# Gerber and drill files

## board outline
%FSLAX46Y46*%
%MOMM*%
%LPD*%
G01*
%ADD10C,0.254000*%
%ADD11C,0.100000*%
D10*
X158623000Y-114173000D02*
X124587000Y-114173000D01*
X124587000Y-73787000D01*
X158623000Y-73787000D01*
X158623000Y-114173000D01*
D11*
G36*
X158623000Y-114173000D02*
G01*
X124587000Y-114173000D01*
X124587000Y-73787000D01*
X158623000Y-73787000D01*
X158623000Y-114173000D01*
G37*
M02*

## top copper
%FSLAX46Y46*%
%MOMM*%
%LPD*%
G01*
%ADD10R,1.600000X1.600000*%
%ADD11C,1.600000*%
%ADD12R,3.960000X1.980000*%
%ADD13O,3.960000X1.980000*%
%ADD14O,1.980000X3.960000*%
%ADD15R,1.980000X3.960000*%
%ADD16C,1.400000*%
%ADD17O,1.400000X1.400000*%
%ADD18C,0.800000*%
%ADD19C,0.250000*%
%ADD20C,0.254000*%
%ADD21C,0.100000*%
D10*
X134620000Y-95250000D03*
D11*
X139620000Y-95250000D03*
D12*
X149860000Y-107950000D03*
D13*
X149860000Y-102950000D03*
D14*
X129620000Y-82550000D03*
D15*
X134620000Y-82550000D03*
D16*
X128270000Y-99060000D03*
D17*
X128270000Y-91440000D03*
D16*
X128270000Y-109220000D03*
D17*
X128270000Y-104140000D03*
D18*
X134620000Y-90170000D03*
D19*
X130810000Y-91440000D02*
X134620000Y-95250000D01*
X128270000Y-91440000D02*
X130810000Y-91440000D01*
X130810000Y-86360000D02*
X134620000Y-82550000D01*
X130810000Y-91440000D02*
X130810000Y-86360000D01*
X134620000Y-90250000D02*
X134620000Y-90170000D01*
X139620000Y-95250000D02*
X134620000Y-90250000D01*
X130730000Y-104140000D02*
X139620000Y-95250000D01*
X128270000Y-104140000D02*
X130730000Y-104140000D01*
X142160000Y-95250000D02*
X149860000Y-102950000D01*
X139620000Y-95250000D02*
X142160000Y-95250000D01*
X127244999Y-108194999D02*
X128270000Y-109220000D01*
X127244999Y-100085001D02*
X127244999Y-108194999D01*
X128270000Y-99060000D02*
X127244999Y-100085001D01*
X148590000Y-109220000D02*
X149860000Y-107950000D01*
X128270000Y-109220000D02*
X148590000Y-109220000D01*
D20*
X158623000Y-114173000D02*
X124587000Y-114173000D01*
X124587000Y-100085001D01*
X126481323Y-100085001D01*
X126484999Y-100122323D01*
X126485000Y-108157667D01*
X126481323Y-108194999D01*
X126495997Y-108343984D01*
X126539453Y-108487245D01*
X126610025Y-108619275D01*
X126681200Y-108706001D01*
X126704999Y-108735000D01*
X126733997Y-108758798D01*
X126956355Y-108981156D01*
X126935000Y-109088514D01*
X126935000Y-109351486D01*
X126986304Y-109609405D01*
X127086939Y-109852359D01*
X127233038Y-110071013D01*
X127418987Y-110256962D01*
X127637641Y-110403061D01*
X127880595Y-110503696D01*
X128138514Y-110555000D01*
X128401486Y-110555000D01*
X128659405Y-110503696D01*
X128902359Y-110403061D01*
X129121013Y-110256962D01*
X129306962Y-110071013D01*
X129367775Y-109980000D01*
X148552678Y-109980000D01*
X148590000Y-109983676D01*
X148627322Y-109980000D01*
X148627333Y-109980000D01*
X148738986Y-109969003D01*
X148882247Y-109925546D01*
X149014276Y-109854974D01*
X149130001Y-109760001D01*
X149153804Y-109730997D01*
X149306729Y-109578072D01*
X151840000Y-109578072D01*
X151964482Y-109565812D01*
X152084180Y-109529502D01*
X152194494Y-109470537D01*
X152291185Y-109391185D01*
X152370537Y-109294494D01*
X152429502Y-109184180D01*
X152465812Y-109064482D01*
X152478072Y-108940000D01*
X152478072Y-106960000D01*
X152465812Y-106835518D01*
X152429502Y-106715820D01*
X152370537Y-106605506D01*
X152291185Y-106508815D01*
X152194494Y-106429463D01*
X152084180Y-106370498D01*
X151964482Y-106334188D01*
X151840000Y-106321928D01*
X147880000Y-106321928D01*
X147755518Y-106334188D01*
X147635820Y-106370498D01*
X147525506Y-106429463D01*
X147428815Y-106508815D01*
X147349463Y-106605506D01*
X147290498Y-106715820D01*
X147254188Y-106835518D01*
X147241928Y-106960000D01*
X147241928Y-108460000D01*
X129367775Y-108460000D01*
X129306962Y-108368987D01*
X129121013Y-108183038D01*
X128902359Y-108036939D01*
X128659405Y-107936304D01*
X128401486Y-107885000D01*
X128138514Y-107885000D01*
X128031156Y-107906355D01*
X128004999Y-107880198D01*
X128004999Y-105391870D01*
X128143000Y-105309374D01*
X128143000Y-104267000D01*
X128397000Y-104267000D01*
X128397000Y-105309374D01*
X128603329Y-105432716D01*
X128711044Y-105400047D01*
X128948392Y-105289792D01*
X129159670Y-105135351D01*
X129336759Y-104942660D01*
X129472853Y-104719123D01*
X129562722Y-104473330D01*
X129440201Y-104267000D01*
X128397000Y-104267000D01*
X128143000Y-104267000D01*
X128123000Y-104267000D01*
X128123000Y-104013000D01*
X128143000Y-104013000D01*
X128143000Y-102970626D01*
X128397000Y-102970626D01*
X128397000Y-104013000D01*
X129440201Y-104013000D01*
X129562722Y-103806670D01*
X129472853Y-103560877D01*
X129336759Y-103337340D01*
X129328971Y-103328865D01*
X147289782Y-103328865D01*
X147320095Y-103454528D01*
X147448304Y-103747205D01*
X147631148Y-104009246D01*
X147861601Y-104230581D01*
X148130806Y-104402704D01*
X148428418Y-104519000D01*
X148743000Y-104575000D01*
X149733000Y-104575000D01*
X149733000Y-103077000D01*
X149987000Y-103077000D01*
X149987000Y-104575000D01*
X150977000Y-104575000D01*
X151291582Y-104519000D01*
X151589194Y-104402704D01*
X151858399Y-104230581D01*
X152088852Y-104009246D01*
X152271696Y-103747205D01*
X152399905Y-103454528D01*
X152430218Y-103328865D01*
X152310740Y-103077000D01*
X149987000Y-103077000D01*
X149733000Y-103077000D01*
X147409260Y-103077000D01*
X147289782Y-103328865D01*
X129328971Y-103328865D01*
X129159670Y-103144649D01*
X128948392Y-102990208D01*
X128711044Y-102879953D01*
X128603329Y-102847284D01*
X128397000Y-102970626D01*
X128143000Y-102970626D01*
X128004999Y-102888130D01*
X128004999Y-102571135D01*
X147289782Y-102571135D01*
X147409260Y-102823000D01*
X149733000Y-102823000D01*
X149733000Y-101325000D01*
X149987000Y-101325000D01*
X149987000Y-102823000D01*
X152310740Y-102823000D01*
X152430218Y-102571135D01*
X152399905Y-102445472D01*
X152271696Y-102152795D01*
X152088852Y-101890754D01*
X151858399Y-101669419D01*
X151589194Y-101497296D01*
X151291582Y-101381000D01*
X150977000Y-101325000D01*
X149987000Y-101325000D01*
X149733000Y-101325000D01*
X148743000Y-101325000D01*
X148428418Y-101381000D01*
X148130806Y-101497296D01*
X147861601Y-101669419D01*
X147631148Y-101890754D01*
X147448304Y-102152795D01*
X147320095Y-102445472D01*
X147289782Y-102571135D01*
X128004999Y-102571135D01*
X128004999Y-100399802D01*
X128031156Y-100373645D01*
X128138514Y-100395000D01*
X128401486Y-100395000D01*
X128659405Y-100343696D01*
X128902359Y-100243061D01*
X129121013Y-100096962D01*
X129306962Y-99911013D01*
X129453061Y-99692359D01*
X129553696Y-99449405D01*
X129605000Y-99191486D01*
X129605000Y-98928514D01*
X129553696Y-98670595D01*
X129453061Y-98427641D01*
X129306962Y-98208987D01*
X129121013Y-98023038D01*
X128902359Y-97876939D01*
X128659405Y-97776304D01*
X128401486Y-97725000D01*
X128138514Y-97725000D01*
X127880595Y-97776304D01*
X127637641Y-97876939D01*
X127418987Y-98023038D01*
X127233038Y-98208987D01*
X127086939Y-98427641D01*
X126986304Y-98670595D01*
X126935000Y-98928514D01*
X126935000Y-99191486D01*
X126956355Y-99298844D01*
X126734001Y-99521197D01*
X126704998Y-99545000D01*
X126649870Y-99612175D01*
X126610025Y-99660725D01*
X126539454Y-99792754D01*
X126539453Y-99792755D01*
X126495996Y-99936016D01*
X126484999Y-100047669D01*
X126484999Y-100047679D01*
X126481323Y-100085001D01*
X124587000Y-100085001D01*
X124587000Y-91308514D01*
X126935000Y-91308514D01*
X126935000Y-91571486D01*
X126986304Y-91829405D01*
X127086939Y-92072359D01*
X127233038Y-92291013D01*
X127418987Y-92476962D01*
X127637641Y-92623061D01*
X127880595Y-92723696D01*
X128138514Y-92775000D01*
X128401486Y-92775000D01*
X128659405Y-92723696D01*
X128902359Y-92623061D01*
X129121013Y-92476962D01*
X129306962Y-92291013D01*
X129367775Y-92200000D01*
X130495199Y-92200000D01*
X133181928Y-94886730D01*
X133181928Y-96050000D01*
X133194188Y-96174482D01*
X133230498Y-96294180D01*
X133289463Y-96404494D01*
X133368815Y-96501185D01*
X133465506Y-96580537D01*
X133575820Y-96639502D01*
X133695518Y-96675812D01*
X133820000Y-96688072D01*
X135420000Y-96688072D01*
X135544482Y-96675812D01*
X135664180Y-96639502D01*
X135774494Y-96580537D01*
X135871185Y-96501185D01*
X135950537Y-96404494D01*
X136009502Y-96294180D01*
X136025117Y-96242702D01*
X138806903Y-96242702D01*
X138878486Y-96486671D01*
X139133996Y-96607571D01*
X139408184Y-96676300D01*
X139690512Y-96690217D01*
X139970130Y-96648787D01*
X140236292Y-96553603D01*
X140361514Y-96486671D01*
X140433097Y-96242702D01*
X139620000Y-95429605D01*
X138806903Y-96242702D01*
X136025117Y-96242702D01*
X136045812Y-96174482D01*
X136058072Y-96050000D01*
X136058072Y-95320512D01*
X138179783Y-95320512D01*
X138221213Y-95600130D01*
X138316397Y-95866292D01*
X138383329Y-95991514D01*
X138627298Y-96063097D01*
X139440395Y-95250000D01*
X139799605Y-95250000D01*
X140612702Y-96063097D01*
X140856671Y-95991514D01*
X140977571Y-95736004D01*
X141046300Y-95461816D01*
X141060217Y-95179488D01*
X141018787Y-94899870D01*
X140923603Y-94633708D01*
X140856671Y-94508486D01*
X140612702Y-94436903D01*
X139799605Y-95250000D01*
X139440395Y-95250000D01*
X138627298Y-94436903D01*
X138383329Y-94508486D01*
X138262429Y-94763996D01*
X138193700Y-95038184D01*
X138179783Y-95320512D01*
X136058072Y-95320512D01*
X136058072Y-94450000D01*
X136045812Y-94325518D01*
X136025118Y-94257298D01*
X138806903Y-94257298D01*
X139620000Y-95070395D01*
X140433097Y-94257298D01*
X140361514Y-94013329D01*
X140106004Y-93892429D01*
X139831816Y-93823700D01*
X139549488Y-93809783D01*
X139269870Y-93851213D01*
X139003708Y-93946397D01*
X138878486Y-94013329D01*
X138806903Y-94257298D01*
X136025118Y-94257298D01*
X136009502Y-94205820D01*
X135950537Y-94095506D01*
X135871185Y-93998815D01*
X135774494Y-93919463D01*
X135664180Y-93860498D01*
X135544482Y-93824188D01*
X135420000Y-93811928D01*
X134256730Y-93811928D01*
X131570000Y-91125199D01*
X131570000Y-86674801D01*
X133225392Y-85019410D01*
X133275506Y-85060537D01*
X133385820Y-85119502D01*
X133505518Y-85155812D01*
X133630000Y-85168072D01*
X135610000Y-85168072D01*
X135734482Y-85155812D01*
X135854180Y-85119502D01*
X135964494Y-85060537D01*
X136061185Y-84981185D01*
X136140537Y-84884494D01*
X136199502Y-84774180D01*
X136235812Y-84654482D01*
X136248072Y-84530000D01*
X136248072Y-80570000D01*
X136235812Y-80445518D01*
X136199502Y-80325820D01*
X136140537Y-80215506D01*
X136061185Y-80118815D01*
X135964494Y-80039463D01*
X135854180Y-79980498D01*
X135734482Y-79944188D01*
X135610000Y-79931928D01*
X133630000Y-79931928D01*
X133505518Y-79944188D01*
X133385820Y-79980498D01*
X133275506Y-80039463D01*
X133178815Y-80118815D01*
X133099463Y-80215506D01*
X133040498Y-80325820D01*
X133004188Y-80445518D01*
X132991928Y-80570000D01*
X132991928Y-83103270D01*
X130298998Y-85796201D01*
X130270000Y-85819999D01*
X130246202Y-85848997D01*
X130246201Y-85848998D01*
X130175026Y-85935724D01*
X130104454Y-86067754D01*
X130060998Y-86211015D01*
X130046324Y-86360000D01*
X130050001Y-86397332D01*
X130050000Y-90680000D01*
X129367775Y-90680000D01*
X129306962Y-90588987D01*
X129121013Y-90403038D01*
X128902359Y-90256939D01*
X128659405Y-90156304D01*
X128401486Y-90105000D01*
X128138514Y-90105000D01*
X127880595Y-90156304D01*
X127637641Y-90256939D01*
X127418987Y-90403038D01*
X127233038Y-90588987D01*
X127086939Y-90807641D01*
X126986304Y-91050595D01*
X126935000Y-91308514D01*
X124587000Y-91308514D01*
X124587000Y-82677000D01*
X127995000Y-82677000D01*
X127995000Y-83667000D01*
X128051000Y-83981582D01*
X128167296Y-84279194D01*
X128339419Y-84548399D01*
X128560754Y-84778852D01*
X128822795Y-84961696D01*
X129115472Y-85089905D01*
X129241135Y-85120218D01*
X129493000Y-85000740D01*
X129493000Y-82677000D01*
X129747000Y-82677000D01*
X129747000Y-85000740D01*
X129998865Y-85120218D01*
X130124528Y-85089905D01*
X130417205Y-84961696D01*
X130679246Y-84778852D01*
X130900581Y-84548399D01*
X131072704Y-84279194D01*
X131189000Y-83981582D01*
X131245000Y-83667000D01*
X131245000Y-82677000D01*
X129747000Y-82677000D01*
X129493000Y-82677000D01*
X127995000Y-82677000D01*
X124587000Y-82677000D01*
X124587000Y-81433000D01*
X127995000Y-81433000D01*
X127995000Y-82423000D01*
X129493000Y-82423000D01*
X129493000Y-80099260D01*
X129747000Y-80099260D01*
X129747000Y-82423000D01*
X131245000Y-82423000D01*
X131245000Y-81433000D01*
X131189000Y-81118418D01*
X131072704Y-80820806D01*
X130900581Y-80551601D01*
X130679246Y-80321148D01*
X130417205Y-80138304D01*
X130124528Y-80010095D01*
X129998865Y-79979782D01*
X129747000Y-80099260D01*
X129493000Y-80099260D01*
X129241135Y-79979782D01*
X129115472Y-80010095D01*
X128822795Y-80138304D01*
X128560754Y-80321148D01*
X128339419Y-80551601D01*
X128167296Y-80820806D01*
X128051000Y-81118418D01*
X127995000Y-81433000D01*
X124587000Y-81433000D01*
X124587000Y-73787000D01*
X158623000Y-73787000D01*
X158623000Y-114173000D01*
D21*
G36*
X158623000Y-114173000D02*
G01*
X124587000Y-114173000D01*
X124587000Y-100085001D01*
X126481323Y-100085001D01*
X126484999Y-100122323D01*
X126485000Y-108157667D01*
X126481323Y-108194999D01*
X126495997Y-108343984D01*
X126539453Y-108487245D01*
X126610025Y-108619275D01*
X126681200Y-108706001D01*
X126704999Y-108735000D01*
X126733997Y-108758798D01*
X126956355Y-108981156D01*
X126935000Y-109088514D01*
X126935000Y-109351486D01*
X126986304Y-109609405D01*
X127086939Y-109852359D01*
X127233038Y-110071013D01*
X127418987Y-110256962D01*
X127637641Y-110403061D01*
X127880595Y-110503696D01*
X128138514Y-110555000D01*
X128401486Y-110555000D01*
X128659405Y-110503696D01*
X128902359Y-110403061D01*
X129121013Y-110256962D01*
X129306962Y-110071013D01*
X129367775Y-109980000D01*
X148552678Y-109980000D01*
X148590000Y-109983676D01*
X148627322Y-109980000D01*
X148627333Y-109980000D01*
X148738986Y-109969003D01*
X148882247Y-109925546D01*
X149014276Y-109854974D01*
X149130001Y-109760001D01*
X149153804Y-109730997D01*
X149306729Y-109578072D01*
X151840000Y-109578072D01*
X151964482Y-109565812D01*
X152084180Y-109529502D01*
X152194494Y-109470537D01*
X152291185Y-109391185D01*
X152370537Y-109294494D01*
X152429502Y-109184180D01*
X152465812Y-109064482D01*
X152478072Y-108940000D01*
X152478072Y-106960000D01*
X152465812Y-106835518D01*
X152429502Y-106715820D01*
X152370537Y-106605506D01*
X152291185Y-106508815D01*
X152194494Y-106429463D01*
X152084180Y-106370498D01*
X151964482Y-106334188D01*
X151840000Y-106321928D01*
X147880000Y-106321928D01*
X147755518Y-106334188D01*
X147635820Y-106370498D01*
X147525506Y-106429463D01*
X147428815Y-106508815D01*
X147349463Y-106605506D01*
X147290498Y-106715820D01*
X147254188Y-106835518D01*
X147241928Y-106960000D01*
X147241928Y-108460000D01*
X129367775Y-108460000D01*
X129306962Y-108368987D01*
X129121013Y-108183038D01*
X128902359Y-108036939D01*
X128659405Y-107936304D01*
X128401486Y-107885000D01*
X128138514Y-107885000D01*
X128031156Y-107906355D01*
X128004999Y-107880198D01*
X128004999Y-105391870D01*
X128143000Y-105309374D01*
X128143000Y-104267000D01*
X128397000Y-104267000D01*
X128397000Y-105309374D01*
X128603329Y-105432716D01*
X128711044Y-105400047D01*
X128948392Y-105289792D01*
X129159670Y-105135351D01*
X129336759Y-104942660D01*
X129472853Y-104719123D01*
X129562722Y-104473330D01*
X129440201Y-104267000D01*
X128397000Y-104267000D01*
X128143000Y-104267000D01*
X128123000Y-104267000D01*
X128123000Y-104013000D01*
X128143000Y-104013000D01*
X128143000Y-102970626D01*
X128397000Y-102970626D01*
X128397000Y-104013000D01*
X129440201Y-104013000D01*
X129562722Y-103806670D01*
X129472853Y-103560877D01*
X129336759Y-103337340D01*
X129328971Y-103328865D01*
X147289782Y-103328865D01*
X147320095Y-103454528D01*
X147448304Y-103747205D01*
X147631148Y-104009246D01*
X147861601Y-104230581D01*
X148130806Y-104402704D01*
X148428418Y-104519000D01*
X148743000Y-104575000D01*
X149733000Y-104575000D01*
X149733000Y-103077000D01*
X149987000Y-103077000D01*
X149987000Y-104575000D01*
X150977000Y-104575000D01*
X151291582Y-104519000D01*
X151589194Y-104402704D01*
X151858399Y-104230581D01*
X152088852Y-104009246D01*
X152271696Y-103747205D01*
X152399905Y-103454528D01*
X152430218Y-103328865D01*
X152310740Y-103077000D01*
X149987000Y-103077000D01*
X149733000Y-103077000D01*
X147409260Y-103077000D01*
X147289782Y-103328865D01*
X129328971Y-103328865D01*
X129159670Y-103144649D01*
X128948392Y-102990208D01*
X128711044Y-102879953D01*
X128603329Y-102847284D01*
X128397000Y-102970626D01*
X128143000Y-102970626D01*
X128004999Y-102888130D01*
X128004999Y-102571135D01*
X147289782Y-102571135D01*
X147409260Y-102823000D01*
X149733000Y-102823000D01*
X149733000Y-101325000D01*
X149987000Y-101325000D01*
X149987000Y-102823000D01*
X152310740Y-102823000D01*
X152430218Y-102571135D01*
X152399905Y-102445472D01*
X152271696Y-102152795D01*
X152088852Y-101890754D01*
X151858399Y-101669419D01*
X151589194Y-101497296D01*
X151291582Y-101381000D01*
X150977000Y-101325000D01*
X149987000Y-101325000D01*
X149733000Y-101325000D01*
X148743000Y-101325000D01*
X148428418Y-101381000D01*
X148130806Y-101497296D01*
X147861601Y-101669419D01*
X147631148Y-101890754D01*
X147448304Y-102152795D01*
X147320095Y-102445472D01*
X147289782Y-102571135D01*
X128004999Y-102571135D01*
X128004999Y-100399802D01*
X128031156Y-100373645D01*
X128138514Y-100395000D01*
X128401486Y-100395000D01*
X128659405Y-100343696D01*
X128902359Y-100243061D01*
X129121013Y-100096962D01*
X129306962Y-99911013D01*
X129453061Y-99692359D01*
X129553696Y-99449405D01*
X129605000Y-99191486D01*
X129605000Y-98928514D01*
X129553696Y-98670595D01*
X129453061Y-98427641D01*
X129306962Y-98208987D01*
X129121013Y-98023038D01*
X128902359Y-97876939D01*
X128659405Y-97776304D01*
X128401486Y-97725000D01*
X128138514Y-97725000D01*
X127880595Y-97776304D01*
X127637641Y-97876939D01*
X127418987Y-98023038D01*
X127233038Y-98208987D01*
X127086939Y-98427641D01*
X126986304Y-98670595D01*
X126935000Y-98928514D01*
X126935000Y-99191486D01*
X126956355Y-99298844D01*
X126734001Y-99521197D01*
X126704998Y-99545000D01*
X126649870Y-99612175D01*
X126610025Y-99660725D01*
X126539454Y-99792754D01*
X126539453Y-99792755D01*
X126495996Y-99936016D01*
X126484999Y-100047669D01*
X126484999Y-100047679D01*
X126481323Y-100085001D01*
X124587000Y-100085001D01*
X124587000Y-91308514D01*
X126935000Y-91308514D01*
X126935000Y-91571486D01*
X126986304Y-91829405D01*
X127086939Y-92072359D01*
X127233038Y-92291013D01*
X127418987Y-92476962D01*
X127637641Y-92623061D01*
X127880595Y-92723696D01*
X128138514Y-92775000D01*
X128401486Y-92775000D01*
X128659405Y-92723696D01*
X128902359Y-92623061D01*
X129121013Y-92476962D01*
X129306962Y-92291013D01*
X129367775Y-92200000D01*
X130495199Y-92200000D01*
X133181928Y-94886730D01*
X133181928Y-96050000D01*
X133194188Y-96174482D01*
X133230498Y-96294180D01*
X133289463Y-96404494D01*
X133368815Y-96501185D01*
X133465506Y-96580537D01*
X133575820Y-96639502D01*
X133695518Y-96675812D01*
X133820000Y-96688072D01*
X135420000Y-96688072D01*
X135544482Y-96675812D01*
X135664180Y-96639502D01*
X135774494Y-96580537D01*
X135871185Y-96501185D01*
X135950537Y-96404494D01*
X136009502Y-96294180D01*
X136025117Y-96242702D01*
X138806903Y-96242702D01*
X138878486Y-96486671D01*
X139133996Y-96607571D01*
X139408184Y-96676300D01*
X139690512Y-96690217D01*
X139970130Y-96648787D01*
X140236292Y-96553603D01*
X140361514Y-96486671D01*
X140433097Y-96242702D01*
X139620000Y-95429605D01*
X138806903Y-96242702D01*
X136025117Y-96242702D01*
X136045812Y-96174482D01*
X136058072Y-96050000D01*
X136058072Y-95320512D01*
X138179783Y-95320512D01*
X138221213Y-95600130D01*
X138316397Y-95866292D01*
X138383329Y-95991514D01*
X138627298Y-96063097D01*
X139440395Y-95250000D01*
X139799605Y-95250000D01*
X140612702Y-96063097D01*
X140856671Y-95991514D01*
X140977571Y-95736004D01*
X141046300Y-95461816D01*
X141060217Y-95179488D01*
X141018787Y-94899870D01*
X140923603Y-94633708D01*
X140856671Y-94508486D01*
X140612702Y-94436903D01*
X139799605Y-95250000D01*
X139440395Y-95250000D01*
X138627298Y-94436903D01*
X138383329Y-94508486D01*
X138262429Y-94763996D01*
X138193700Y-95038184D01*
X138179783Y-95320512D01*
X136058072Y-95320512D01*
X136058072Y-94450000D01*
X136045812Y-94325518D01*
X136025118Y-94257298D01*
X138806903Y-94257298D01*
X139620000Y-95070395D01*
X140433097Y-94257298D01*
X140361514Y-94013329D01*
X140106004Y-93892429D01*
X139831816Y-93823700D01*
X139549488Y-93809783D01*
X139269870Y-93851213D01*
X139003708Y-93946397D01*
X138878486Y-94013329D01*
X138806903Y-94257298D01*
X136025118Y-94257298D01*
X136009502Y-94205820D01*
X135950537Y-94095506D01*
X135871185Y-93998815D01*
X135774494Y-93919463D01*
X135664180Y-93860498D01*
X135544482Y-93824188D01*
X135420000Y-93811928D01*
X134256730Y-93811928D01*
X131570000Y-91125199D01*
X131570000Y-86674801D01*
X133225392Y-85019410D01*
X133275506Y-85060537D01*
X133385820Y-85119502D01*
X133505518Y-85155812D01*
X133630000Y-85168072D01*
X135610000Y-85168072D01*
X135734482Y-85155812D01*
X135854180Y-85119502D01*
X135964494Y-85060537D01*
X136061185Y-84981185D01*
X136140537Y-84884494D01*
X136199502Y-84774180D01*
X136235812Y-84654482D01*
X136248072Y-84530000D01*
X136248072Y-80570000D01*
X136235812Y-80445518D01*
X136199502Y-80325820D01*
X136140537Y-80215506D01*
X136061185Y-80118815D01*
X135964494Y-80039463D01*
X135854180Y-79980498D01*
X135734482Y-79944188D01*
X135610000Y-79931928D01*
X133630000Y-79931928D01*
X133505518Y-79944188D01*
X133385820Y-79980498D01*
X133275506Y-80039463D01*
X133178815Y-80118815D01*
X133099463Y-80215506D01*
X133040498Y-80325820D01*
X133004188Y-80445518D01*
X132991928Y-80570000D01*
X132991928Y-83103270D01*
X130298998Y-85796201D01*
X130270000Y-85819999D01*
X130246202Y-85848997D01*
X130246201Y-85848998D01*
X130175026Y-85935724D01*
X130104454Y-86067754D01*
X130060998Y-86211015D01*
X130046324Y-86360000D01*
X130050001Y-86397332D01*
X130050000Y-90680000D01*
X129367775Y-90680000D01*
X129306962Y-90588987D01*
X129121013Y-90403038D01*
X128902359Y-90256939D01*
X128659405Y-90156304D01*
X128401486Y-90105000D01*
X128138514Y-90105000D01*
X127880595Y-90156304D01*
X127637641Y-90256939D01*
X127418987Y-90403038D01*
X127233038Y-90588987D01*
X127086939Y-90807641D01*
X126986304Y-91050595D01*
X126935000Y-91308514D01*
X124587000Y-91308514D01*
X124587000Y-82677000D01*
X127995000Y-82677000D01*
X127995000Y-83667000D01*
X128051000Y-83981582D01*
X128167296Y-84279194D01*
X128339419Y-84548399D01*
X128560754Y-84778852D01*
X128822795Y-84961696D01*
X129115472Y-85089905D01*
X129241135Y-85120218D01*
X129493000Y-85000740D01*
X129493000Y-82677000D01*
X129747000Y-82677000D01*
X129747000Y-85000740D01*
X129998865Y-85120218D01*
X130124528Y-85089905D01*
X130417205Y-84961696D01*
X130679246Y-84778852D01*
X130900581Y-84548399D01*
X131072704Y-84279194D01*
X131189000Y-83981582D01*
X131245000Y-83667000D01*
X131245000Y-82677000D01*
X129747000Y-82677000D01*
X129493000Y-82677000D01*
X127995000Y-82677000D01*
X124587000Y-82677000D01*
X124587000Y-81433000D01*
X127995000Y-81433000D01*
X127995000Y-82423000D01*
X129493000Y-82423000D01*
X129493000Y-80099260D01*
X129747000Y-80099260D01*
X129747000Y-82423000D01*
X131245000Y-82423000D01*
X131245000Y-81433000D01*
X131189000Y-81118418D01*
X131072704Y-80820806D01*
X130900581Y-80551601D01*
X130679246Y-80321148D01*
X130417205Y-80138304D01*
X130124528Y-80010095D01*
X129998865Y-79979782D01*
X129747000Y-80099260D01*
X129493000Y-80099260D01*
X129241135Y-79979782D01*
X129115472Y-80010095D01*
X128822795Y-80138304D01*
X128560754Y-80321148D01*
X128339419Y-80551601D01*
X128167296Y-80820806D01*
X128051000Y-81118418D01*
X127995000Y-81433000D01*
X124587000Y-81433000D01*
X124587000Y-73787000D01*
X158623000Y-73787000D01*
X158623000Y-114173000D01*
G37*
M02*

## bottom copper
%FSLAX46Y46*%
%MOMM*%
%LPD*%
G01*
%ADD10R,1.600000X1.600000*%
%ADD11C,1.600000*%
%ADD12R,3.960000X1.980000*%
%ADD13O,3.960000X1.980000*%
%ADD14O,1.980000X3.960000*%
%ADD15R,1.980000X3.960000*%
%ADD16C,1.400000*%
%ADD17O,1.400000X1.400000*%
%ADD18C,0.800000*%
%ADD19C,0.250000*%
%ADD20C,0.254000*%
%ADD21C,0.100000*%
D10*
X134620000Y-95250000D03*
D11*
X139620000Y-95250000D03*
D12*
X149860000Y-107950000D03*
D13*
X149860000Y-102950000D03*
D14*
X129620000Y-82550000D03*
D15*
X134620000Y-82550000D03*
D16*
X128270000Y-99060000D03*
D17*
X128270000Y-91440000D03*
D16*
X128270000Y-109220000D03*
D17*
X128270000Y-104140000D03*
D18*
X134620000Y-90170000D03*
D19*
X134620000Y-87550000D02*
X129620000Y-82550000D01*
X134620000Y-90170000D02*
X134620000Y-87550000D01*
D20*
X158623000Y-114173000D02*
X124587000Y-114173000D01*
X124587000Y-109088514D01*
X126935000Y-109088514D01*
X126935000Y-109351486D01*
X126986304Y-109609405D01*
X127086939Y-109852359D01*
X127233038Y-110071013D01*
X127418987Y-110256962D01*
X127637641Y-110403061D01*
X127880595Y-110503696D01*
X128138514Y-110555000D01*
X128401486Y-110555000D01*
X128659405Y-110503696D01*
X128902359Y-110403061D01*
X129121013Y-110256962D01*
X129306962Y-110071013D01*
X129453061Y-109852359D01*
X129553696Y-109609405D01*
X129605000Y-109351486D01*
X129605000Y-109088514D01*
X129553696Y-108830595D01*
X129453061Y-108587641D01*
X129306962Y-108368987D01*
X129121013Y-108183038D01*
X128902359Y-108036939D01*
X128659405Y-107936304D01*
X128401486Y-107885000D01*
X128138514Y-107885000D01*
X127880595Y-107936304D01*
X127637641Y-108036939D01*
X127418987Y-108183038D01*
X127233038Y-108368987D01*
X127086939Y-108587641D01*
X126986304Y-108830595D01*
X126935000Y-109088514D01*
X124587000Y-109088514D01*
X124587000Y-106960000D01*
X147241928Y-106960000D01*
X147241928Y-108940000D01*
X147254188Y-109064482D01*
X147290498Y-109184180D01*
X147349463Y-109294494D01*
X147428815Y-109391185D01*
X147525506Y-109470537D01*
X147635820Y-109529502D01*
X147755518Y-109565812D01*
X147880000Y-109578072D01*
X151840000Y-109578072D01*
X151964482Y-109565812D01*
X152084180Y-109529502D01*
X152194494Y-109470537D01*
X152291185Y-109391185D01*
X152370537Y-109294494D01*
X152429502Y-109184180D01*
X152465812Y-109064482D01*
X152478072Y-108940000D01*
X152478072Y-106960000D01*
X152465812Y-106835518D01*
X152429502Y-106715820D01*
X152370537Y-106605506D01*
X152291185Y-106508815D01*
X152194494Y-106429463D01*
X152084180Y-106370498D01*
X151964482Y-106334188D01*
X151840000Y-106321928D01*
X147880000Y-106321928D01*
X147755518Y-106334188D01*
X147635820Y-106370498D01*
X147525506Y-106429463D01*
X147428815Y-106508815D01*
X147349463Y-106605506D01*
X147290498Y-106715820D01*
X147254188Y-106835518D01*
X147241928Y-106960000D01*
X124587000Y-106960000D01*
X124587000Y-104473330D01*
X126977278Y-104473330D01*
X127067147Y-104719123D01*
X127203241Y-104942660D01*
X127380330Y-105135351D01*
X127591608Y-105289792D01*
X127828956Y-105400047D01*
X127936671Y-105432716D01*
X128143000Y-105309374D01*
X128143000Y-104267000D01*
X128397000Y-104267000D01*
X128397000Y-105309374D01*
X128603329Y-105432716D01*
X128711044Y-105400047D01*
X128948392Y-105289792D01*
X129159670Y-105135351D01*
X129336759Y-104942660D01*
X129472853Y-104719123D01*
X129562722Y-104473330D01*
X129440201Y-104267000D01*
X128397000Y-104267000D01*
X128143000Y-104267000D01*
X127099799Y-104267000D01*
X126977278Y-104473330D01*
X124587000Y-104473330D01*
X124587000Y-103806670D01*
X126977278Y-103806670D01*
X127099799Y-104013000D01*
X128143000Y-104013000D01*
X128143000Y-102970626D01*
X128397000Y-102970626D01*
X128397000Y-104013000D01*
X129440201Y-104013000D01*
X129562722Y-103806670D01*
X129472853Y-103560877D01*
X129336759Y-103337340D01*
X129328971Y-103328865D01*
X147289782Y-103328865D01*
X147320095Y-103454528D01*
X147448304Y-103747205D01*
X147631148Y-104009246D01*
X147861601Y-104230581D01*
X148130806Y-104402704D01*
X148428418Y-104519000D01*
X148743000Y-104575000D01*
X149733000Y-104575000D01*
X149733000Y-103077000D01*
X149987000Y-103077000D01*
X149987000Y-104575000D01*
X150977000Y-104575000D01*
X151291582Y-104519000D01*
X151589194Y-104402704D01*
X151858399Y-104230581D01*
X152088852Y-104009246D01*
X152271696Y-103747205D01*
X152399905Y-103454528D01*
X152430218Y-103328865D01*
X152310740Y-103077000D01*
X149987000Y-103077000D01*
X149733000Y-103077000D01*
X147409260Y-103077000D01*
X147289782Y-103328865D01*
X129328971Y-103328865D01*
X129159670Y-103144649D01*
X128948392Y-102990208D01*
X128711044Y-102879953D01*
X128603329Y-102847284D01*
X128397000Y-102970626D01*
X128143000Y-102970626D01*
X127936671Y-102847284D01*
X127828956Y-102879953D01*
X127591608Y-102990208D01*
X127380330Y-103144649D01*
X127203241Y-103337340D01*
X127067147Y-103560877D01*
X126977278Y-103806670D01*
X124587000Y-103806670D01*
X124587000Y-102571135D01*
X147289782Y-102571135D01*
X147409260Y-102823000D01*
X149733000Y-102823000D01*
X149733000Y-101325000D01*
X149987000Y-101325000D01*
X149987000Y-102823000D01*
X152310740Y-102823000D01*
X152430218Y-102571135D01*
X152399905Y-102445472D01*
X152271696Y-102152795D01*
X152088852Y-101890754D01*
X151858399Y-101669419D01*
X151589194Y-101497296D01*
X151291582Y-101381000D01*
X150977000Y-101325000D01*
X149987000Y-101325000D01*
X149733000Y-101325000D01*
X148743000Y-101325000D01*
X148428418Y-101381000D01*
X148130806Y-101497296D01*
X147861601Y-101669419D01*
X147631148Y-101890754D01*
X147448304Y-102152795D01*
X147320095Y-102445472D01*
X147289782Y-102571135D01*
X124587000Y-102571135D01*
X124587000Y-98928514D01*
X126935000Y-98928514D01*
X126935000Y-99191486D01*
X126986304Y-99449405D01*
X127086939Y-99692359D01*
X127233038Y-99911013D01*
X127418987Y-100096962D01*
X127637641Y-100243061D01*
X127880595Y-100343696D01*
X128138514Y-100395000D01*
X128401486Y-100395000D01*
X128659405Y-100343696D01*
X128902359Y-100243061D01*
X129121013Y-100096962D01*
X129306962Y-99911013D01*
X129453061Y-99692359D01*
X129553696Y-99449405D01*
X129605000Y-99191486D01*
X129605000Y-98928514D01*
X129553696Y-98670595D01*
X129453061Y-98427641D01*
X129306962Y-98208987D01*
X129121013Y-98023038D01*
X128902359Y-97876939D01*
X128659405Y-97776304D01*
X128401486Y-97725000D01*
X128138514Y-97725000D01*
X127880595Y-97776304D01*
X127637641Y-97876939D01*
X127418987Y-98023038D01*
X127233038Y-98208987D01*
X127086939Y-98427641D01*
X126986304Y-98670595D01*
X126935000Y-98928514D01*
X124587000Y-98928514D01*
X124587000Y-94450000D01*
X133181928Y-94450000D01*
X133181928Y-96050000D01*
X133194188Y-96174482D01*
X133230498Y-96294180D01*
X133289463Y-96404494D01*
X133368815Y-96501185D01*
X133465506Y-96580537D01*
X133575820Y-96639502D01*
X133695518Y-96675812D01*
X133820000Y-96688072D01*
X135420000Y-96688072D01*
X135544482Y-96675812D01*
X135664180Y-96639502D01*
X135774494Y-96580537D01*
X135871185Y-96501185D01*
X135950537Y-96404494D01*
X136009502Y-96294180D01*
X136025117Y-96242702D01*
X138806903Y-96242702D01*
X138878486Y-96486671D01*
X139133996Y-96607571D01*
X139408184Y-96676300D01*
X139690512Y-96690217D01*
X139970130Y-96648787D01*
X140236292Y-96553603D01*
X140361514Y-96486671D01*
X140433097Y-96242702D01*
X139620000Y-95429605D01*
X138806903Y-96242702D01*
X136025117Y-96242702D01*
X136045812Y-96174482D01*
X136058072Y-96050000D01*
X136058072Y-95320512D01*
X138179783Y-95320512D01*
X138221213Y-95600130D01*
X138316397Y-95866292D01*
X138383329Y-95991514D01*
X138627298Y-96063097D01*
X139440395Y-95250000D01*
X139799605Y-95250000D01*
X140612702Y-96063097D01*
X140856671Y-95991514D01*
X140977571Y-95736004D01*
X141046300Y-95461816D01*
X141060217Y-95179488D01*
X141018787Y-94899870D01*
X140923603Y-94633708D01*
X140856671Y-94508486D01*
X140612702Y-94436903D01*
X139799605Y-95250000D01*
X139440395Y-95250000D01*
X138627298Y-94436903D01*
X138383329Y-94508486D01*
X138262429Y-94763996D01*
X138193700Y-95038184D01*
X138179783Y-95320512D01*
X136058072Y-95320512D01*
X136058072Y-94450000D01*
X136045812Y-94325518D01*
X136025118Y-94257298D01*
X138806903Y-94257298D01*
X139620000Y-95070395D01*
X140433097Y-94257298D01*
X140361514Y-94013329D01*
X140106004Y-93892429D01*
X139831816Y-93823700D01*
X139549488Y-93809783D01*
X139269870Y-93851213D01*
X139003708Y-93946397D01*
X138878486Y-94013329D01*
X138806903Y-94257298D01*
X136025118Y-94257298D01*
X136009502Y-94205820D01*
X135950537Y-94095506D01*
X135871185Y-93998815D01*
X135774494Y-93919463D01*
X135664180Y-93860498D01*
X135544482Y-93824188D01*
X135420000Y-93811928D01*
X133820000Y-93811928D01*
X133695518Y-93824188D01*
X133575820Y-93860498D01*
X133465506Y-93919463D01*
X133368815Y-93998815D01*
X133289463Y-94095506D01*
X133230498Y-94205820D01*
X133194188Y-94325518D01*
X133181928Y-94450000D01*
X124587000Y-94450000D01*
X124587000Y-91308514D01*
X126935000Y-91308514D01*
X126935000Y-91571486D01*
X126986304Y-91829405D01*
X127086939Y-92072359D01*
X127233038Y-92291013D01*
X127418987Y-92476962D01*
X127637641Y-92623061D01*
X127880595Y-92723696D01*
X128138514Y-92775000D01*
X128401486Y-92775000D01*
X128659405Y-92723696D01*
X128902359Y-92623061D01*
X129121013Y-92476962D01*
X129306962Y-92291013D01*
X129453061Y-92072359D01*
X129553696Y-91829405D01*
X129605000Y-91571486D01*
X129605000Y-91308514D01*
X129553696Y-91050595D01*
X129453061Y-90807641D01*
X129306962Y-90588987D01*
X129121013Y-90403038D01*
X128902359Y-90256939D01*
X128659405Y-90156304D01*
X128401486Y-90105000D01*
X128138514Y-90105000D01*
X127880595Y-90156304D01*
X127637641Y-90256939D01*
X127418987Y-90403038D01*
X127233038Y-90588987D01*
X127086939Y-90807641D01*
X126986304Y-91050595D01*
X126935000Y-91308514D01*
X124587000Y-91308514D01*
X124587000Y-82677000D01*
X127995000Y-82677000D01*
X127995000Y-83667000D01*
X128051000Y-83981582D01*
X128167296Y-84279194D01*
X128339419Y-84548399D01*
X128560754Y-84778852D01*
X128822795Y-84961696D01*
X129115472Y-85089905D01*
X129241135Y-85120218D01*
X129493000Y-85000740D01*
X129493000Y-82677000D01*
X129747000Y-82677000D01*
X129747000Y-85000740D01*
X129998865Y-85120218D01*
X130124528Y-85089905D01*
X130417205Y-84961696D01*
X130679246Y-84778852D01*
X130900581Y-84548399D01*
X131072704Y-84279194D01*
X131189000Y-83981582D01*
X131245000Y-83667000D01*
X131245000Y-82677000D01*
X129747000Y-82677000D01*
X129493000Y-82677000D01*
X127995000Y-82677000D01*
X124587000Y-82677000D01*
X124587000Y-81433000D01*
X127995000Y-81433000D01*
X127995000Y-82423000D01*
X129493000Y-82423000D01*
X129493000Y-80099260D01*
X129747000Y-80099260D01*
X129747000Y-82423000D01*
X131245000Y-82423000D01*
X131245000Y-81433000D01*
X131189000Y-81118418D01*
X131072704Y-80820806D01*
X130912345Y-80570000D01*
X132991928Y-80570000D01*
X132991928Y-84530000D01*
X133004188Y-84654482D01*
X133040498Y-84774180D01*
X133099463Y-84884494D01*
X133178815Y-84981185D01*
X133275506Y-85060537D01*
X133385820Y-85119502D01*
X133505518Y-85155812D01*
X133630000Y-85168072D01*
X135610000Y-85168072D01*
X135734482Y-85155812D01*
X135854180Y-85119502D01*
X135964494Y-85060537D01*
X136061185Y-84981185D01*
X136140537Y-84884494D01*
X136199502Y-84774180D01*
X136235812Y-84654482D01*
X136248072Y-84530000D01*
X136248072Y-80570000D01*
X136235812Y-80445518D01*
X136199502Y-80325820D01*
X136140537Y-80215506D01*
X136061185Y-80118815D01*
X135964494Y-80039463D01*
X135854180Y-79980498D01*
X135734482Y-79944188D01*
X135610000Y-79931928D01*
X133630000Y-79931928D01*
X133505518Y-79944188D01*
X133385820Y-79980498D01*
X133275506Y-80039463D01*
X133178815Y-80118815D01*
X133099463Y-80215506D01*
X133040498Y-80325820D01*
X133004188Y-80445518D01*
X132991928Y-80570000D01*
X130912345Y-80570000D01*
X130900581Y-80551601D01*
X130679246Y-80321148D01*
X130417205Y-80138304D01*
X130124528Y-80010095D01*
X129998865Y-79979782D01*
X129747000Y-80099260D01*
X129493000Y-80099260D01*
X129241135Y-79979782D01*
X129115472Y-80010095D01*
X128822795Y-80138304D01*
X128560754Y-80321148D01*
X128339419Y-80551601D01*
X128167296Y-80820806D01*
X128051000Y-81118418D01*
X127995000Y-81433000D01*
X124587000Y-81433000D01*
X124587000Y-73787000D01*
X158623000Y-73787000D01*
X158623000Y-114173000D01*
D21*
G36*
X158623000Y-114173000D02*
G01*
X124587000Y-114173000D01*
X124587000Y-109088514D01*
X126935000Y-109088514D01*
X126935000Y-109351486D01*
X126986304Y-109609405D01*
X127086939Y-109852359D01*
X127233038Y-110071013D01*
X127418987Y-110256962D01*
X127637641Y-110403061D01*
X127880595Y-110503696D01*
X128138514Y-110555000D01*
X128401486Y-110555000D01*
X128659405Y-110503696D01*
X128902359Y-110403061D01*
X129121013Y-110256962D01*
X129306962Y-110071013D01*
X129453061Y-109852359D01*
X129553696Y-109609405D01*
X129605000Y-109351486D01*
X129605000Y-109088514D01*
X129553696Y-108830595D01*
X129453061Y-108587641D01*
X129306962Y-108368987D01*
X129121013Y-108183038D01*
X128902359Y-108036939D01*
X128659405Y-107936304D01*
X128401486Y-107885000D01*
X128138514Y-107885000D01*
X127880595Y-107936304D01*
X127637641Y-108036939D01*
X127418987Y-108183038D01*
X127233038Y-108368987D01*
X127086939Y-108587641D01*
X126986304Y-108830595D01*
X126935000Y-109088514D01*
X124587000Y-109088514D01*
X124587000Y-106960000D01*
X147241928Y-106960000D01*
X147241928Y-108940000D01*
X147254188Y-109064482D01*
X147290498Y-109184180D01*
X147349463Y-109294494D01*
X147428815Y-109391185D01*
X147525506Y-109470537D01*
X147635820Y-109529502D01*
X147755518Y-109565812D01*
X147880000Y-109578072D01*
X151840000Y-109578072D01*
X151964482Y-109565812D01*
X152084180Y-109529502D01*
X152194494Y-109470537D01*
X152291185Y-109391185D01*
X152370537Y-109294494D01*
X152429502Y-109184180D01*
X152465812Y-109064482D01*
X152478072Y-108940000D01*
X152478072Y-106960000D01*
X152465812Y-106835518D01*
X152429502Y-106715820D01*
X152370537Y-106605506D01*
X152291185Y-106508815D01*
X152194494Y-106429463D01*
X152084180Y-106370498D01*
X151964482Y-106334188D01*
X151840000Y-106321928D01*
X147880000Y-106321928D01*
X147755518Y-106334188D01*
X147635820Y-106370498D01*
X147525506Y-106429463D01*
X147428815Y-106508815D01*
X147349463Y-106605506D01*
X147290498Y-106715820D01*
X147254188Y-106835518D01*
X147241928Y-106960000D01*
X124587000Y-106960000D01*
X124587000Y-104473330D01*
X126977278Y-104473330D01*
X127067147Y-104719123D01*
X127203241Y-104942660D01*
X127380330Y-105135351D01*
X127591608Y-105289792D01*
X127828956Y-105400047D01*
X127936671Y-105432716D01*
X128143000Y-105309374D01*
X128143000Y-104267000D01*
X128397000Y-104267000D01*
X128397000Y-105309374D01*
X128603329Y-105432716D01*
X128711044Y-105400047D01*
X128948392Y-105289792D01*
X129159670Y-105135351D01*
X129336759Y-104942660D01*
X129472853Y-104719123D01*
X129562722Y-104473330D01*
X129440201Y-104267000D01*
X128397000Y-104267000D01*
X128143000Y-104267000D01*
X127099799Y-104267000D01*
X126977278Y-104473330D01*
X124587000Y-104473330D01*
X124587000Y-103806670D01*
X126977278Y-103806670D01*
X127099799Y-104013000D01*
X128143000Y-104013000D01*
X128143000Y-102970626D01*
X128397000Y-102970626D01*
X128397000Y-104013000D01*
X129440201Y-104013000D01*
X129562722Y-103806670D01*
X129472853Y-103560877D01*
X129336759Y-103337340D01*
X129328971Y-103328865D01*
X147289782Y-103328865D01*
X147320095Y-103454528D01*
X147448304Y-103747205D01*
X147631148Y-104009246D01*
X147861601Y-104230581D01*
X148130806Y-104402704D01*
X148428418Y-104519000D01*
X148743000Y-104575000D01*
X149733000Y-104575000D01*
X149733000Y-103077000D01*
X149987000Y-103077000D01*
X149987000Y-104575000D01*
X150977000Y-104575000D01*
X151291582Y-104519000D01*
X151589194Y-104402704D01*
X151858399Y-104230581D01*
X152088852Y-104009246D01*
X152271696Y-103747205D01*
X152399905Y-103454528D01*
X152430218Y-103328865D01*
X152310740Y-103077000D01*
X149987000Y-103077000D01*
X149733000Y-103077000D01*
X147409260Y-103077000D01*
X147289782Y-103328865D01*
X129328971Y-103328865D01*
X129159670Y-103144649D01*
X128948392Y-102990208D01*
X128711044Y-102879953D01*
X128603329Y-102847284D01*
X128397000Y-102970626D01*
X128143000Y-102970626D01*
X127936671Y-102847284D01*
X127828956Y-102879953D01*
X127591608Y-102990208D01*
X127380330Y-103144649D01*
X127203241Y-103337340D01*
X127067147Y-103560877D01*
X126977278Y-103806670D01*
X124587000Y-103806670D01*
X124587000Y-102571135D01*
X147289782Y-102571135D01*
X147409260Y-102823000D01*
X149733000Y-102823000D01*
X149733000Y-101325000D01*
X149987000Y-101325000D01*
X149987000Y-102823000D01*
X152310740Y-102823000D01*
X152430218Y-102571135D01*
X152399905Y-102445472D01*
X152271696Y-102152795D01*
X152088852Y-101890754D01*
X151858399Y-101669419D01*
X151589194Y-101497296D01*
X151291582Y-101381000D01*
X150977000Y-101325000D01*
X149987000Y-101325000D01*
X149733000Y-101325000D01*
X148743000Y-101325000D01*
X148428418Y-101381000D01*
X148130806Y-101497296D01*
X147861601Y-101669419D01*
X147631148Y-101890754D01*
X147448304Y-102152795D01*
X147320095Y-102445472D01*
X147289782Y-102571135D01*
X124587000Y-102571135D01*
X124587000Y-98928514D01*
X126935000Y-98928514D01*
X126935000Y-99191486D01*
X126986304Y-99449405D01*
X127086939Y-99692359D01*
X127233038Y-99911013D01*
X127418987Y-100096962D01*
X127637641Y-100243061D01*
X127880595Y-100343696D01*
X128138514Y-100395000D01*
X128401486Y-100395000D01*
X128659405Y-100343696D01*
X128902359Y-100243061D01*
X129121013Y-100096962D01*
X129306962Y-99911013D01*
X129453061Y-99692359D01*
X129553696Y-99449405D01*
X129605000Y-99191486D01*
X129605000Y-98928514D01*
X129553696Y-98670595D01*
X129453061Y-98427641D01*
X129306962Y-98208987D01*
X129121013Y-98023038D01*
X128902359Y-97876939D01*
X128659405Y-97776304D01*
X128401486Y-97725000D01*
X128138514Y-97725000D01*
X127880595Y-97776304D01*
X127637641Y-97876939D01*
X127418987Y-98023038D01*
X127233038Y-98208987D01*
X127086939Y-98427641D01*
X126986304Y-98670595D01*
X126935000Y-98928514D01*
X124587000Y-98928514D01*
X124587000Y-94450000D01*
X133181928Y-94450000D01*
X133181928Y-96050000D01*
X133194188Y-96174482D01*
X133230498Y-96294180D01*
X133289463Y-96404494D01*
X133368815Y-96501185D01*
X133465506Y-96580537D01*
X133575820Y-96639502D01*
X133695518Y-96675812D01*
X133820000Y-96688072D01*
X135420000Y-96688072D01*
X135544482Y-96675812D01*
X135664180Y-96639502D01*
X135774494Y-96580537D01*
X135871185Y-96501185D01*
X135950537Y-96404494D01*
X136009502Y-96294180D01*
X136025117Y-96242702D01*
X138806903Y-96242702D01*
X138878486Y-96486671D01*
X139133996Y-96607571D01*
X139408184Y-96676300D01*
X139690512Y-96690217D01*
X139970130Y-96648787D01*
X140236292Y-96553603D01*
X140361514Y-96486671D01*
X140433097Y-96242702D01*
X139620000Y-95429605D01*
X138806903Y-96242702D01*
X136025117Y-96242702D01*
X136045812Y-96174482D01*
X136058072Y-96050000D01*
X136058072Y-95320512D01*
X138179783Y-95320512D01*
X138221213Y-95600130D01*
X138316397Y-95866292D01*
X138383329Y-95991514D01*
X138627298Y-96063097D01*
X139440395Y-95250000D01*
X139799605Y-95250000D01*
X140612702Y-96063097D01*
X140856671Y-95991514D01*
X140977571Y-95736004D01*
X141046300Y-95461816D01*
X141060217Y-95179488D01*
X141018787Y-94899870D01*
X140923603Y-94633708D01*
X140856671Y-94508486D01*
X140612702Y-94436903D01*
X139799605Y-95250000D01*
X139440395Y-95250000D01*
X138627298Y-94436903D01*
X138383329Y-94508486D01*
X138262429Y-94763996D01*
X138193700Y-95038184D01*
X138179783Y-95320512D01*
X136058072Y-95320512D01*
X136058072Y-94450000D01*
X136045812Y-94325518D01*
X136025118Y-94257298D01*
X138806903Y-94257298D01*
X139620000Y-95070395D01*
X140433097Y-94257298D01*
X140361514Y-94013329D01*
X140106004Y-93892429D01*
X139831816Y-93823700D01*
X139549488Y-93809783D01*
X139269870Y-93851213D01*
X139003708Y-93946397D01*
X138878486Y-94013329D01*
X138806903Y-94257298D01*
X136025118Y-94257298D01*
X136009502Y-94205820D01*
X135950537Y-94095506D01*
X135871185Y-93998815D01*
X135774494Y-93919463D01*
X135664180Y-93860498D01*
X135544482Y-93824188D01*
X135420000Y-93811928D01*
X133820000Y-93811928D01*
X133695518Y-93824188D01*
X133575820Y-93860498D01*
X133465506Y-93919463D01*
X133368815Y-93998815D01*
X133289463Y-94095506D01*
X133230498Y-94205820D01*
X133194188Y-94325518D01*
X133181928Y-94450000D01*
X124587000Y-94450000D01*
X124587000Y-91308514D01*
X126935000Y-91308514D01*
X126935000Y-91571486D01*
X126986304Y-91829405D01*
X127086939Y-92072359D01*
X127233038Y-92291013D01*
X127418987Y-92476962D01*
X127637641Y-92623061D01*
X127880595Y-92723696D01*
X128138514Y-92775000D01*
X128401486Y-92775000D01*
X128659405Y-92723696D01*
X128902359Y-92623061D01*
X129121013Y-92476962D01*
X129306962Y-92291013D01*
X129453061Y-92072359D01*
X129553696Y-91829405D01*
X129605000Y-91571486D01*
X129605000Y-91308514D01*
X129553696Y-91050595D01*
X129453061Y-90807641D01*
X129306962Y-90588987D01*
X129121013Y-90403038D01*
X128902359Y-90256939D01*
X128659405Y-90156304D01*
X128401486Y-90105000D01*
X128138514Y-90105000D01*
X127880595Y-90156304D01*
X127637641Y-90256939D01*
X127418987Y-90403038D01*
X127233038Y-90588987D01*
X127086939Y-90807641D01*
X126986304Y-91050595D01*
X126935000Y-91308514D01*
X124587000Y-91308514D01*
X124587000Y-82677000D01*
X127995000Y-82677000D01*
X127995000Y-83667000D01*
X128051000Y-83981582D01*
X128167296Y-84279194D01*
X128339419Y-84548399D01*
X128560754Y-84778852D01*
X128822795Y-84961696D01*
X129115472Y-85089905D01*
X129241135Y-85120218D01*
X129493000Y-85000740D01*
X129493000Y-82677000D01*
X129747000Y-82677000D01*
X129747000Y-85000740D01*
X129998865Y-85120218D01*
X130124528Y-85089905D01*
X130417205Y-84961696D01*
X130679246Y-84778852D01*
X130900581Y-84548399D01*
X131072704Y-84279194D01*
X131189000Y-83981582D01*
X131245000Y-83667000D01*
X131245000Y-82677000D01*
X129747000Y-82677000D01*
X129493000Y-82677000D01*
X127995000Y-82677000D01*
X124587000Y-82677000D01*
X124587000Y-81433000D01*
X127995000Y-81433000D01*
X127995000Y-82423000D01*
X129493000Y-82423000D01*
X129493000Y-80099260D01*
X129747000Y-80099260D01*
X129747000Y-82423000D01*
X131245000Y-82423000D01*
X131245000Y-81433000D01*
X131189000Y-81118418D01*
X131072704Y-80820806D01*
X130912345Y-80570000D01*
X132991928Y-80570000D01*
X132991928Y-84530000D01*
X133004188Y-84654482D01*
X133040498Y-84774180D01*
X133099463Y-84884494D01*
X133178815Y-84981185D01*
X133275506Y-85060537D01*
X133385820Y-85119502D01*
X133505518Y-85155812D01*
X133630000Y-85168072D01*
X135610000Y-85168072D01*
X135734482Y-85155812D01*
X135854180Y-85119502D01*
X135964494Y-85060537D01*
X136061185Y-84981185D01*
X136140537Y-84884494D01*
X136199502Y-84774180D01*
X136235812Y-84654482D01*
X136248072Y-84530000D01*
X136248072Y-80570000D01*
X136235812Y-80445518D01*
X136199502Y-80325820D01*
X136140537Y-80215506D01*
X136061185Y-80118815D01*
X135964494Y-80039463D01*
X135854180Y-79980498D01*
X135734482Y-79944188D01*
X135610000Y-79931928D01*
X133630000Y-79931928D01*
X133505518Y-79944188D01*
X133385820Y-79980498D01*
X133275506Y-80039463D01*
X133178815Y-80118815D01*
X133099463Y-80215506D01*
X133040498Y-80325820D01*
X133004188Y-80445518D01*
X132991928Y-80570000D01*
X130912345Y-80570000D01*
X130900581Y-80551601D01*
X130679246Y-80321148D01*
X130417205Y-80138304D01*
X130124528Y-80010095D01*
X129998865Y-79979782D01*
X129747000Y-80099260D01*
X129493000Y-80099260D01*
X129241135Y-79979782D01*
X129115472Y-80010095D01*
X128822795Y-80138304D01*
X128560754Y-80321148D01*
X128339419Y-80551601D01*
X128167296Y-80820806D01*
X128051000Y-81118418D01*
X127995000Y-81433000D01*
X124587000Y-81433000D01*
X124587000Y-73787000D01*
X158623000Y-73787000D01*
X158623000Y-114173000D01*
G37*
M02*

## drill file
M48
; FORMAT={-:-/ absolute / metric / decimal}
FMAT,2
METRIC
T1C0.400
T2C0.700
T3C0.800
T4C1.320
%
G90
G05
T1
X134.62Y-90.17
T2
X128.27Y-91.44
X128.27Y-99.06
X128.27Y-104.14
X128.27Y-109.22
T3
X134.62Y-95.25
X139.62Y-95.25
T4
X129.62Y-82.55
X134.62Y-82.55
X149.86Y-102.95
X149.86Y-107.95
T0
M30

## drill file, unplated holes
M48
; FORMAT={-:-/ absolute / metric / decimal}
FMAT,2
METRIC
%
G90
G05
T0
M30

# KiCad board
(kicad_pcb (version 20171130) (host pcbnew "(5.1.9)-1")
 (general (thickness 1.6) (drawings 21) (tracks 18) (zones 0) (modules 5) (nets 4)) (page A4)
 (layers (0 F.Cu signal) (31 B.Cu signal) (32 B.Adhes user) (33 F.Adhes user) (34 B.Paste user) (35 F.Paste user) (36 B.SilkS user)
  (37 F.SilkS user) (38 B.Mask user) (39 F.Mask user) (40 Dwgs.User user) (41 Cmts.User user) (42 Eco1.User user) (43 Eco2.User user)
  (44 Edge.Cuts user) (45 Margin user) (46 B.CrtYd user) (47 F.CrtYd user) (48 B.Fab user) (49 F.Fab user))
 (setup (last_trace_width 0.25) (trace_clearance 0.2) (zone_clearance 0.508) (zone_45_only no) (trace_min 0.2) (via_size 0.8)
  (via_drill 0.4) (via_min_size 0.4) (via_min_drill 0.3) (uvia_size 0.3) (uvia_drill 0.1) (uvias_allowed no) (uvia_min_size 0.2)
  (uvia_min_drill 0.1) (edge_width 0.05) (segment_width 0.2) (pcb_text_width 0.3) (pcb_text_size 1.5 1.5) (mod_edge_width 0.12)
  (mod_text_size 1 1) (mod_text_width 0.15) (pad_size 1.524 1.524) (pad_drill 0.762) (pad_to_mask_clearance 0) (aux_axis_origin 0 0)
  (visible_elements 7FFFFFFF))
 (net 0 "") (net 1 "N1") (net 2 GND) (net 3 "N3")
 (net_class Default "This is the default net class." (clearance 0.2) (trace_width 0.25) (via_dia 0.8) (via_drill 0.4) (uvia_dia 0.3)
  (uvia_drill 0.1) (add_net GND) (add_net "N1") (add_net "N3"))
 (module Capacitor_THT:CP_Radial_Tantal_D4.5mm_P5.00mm (layer F.Cu) (at 134.62 95.25)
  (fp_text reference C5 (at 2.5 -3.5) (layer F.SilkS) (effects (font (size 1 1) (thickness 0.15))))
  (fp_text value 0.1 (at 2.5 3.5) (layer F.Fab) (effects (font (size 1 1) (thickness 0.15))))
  (pad 1 thru_hole rect (at 0 0) (size 1.6 1.6) (drill 0.8) (layers *.Cu *.Mask) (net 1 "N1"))
  (pad 2 thru_hole circle (at 5 0) (size 1.6 1.6) (drill 0.8) (layers *.Cu *.Mask) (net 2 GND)))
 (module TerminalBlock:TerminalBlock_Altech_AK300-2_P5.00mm (layer F.Cu) (at 149.86 107.95 90)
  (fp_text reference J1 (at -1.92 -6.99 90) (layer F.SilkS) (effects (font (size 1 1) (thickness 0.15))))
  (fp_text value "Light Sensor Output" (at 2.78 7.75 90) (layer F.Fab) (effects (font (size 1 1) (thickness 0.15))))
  (pad 1 thru_hole rect (at 0 0 90) (size 1.98 3.96) (drill 1.32) (layers *.Cu *.Mask) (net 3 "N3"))
  (pad 2 thru_hole oval (at 5 0 90) (size 1.98 3.96) (drill 1.32) (layers *.Cu *.Mask) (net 2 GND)))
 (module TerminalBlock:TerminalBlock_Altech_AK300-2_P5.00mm (layer F.Cu) (at 134.62 82.55 180)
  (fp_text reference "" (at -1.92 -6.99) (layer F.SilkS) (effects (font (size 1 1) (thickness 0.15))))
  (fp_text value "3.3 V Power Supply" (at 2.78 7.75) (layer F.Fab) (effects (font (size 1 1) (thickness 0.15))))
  (pad 2 thru_hole oval (at 5 0 180) (size 1.98 3.96) (drill 1.32) (layers *.Cu *.Mask) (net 2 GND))
  (pad 1 thru_hole rect (at 0 0 180) (size 1.98 3.96) (drill 1.32) (layers *.Cu *.Mask) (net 1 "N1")))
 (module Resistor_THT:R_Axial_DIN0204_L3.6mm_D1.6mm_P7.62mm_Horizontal (layer F.Cu) (at 128.27 99.06 90)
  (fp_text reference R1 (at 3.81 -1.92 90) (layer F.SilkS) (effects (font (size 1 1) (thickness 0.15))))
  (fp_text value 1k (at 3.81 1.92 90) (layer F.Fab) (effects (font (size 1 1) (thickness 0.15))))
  (pad 1 thru_hole circle (at 0 0 90) (size 1.4 1.4) (drill 0.7) (layers *.Cu *.Mask) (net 3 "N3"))
  (pad 2 thru_hole oval (at 7.62 0 90) (size 1.4 1.4) (drill 0.7) (layers *.Cu *.Mask) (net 1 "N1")))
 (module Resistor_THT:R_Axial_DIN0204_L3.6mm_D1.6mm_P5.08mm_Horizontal (layer F.Cu) (at 128.27 109.22 90)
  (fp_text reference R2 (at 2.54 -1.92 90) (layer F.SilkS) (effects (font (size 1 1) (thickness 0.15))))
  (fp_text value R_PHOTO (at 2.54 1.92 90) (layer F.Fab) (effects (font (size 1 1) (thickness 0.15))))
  (pad 1 thru_hole circle (at 0 0 90) (size 1.4 1.4) (drill 0.7) (layers *.Cu *.Mask) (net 3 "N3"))
  (pad 2 thru_hole oval (at 5.08 0 90) (size 1.4 1.4) (drill 0.7) (layers *.Cu *.Mask) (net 2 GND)))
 (segment (start 130.81 91.44) (end 134.62 95.25) (width 0.25) (layer F.Cu) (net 1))
 (segment (start 128.27 91.44) (end 130.81 91.44) (width 0.25) (layer F.Cu) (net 1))
 (segment (start 130.81 86.36) (end 134.62 82.55) (width 0.25) (layer F.Cu) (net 1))
 (segment (start 130.81 91.44) (end 130.81 86.36) (width 0.25) (layer F.Cu) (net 1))
 (via (at 134.62 90.17) (size 0.8) (drill 0.4) (layers F.Cu B.Cu) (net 2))
 (segment (start 134.62 90.25) (end 134.62 90.17) (width 0.25) (layer F.Cu) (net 2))
 (segment (start 139.62 95.25) (end 134.62 90.25) (width 0.25) (layer F.Cu) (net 2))
 (segment (start 134.62 87.55) (end 129.62 82.55) (width 0.25) (layer B.Cu) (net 2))
 (segment (start 134.62 90.17) (end 134.62 87.55) (width 0.25) (layer B.Cu) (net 2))
 (segment (start 130.73 104.14) (end 139.62 95.25) (width 0.25) (layer F.Cu) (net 2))
 (segment (start 128.27 104.14) (end 130.73 104.14) (width 0.25) (layer F.Cu) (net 2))
 (segment (start 142.16 95.25) (end 149.86 102.95) (width 0.25) (layer F.Cu) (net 2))
 (segment (start 139.62 95.25) (end 142.16 95.25) (width 0.25) (layer F.Cu) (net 2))
 (segment (start 127.244999 108.194999) (end 128.27 109.22) (width 0.25) (layer F.Cu) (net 3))
 (segment (start 127.244999 100.085001) (end 127.244999 108.194999) (width 0.25) (layer F.Cu) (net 3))
 (segment (start 128.27 99.06) (end 127.244999 100.085001) (width 0.25) (layer F.Cu) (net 3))
 (segment (start 148.59 109.22) (end 149.86 107.95) (width 0.25) (layer F.Cu) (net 3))
 (segment (start 128.27 109.22) (end 148.59 109.22) (width 0.25) (layer F.Cu) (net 3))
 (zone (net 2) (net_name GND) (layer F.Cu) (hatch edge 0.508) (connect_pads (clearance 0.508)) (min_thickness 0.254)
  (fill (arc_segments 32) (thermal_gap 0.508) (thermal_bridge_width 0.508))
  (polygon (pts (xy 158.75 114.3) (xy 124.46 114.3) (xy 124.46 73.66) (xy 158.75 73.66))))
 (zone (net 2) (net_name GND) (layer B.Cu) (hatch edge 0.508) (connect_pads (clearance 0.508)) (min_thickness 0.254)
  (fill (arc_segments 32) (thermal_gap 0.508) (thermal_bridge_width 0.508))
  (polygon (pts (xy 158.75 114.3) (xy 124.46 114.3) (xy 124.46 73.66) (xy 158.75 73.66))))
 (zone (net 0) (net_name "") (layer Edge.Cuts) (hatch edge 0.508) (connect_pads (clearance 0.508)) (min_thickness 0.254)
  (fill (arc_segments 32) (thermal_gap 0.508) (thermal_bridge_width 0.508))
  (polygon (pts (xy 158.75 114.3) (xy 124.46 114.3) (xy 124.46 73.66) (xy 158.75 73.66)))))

